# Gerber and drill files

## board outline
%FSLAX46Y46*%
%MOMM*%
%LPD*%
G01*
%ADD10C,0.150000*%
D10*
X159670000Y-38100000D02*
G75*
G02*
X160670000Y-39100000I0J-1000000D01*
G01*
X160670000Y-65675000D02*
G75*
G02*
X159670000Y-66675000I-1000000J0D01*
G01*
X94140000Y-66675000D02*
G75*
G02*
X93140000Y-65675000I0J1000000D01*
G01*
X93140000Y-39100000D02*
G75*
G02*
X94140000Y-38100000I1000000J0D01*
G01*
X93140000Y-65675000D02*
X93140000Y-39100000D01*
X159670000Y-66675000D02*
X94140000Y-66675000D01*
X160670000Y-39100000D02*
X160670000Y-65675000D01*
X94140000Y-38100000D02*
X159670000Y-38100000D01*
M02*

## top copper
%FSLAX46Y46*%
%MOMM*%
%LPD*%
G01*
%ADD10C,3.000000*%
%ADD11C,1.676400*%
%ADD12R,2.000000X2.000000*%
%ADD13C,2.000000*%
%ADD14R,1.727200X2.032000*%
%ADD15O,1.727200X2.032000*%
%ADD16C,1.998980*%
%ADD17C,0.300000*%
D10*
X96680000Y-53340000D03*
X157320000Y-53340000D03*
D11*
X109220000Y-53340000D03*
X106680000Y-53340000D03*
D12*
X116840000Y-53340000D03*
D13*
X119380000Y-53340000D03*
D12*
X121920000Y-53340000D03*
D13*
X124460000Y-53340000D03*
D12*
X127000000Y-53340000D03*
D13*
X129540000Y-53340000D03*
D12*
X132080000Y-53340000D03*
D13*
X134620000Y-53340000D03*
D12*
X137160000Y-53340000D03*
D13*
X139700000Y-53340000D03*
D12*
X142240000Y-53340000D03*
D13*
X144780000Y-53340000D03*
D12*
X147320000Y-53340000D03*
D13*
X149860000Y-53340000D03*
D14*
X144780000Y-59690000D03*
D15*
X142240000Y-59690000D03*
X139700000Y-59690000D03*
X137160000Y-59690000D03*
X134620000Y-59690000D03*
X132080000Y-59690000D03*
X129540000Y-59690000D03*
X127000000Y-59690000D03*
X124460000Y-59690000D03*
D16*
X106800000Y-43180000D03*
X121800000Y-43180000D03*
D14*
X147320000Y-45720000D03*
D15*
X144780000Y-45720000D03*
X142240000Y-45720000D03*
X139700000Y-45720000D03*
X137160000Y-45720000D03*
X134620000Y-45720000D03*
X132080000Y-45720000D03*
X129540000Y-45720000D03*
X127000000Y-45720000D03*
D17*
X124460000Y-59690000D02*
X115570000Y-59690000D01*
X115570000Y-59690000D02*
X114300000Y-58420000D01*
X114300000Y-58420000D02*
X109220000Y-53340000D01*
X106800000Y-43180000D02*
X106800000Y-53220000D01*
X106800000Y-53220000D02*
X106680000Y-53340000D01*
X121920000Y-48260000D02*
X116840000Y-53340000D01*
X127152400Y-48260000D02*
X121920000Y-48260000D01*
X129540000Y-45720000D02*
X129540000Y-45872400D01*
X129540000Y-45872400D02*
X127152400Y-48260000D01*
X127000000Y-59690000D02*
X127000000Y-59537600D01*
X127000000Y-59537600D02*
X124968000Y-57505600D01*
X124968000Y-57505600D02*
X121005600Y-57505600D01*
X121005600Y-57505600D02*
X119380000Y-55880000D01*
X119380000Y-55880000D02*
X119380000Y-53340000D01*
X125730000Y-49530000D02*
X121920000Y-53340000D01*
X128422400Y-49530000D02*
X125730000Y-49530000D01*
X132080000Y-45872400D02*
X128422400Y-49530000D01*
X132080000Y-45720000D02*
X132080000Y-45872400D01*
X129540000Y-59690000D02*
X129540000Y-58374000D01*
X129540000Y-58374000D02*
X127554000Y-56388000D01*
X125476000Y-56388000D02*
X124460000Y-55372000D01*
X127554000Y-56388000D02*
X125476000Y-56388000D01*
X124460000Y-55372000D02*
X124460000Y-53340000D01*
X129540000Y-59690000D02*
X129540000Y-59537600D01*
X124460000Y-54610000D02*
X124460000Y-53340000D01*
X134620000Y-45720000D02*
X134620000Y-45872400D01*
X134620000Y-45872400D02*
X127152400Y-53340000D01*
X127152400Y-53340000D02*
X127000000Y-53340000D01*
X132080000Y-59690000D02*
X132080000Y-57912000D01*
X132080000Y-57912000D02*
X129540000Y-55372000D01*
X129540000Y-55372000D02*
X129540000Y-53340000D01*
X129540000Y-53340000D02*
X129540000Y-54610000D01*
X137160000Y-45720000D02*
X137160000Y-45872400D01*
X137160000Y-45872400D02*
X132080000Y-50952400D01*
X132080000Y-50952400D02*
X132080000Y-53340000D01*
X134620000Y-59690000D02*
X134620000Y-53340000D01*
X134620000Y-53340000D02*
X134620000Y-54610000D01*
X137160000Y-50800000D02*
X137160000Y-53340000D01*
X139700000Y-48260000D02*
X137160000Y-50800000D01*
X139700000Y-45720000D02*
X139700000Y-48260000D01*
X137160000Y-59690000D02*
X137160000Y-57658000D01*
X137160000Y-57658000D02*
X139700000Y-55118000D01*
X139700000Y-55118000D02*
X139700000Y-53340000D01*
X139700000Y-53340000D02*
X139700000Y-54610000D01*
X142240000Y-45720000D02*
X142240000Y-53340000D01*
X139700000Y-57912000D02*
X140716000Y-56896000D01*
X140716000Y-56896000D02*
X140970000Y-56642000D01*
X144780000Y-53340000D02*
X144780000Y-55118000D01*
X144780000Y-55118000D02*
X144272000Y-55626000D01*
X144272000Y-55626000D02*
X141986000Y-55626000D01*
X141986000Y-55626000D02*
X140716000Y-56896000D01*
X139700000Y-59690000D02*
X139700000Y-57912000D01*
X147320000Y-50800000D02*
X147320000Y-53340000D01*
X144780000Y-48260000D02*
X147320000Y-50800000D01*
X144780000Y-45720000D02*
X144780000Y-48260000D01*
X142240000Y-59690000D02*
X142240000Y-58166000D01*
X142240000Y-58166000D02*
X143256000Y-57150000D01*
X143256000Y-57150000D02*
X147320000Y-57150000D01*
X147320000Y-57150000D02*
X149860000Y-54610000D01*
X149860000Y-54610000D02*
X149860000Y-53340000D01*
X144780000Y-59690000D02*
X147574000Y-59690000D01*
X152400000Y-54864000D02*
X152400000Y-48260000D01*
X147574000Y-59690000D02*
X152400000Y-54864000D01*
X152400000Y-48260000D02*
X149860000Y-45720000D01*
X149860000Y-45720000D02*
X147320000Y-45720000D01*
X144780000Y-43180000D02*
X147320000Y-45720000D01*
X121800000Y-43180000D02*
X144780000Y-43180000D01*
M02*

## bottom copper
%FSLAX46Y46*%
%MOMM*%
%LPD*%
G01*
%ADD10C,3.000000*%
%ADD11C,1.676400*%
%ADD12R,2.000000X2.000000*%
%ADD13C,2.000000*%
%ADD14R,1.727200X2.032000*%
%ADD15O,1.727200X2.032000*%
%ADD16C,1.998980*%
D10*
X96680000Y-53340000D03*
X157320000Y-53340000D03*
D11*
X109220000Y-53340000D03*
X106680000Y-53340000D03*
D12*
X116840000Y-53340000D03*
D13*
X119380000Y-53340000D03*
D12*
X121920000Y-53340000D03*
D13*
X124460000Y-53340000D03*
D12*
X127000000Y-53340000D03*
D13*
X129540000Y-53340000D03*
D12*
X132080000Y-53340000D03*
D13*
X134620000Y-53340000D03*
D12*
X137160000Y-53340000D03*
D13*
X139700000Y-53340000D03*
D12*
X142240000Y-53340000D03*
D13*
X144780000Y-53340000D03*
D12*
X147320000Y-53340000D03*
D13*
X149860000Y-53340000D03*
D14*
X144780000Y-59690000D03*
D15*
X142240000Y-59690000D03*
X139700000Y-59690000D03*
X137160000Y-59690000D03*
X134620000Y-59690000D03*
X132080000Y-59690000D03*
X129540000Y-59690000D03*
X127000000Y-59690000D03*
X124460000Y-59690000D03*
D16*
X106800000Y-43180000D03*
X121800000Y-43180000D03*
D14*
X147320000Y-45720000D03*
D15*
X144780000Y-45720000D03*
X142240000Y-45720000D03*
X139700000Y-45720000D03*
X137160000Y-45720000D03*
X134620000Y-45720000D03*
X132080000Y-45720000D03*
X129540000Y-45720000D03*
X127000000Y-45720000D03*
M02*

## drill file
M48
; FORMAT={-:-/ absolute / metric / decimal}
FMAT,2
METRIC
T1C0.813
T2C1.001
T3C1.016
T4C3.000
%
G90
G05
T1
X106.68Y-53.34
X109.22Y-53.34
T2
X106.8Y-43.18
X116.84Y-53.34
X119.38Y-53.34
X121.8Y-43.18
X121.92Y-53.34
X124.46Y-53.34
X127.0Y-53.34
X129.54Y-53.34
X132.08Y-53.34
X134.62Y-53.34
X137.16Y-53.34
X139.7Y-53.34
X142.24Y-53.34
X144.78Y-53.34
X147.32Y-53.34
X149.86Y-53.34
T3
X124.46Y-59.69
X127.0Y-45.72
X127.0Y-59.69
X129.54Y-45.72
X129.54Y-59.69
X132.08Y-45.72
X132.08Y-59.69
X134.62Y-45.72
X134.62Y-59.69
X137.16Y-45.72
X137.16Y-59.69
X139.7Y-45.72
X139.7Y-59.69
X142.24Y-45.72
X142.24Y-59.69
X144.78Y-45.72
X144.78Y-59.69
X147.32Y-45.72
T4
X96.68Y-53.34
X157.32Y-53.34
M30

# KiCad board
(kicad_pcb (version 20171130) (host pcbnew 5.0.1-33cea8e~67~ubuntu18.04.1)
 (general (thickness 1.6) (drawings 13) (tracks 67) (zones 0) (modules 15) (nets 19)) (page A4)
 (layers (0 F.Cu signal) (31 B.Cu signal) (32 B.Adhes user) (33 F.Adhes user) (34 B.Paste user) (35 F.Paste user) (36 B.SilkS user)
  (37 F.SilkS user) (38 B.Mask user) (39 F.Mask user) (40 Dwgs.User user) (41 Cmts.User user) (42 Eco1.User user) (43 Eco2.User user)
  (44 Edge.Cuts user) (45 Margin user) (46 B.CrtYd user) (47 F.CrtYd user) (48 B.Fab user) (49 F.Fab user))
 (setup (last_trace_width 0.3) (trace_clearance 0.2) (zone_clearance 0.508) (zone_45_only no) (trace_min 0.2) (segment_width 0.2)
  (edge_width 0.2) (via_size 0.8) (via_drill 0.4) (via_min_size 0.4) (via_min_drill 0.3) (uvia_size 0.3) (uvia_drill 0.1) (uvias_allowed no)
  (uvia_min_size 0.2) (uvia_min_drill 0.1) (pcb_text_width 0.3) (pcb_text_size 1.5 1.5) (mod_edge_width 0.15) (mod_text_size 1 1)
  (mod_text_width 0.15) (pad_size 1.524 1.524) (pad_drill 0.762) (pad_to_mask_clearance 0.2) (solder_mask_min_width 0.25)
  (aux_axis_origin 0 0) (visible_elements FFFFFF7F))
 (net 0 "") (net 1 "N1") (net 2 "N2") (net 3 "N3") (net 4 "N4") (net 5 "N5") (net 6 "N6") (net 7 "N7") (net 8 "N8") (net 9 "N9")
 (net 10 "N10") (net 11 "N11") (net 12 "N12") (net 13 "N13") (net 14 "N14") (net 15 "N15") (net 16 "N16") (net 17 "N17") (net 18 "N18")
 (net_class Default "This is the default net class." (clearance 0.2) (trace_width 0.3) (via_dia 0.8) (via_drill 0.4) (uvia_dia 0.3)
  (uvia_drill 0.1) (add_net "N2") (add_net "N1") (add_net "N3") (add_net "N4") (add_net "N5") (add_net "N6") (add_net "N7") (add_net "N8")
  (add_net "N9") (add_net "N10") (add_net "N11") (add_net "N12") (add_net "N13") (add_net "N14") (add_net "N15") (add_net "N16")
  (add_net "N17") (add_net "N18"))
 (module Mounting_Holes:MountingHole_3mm (layer F.Cu) (at 96.68 53.34)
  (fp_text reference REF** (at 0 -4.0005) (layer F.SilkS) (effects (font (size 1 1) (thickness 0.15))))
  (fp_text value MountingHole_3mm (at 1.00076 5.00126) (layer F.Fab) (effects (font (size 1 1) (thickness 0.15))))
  (pad 1 thru_hole circle (at 0 0) (size 3 3) (drill 3) (layers)))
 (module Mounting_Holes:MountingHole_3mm (layer F.Cu) (at 157.32 53.34)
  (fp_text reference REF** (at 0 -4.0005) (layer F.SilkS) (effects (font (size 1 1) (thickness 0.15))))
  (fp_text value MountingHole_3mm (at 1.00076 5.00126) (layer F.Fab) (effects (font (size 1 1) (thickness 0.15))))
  (pad 1 thru_hole circle (at 0 0) (size 3 3) (drill 3) (layers)))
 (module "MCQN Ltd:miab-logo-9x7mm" (layer B.Cu) (at 154.432 61.722 180)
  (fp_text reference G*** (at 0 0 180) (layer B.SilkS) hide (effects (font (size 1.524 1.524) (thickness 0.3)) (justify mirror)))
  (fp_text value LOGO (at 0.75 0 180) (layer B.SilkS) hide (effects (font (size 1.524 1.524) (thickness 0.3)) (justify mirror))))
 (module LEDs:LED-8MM (layer B.Cu) (at 106.68 53.34)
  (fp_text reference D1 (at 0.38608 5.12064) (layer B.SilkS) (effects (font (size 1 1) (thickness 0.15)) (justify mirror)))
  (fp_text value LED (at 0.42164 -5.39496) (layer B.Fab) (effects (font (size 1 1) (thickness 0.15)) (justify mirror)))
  (pad 2 thru_hole circle (at 2.54 0 180) (size 1.6764 1.6764) (drill 0.8128) (layers *.Cu *.Mask B.SilkS) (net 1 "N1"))
  (pad 1 thru_hole circle (at 0 0 180) (size 1.6764 1.6764) (drill 0.8128) (layers *.Cu *.Mask B.SilkS) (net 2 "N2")))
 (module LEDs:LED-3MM (layer B.Cu) (at 116.84 53.34)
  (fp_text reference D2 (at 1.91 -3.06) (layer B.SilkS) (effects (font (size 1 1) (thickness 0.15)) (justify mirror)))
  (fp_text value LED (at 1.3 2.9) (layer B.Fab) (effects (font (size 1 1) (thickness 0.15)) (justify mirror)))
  (pad 1 thru_hole rect (at 0 0 270) (size 2 2) (drill 1.00076) (layers *.Cu *.Mask B.SilkS) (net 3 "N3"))
  (pad 2 thru_hole circle (at 2.54 0) (size 2 2) (drill 1.00076) (layers *.Cu *.Mask B.SilkS) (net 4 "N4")))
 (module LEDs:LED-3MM (layer B.Cu) (at 121.92 53.34)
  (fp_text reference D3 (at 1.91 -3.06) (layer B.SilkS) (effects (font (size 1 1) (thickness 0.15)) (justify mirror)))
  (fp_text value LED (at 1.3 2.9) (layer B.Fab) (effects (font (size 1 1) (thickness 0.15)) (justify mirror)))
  (pad 1 thru_hole rect (at 0 0 270) (size 2 2) (drill 1.00076) (layers *.Cu *.Mask B.SilkS) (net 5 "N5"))
  (pad 2 thru_hole circle (at 2.54 0) (size 2 2) (drill 1.00076) (layers *.Cu *.Mask B.SilkS) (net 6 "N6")))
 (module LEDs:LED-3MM (layer B.Cu) (at 127 53.34)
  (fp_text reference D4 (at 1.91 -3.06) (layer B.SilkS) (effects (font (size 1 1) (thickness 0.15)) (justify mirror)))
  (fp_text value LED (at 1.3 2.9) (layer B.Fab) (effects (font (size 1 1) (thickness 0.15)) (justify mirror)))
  (pad 1 thru_hole rect (at 0 0 270) (size 2 2) (drill 1.00076) (layers *.Cu *.Mask B.SilkS) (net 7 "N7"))
  (pad 2 thru_hole circle (at 2.54 0) (size 2 2) (drill 1.00076) (layers *.Cu *.Mask B.SilkS) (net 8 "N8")))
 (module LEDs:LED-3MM (layer B.Cu) (at 132.08 53.34)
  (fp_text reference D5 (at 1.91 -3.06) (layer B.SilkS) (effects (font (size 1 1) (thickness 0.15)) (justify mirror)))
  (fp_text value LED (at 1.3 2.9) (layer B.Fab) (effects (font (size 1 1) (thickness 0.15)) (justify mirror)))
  (pad 1 thru_hole rect (at 0 0 270) (size 2 2) (drill 1.00076) (layers *.Cu *.Mask B.SilkS) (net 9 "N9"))
  (pad 2 thru_hole circle (at 2.54 0) (size 2 2) (drill 1.00076) (layers *.Cu *.Mask B.SilkS) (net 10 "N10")))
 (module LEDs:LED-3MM (layer B.Cu) (at 137.16 53.34)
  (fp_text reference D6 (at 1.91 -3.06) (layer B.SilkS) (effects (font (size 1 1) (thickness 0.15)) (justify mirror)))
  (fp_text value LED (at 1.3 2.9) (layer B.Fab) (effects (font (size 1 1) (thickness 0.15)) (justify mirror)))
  (pad 1 thru_hole rect (at 0 0 270) (size 2 2) (drill 1.00076) (layers *.Cu *.Mask B.SilkS) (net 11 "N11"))
  (pad 2 thru_hole circle (at 2.54 0) (size 2 2) (drill 1.00076) (layers *.Cu *.Mask B.SilkS) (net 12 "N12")))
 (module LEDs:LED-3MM (layer B.Cu) (at 142.24 53.34)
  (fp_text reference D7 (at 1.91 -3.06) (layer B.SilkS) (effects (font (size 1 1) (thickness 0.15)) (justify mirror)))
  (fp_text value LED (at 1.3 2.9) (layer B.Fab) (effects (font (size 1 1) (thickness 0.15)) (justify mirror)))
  (pad 1 thru_hole rect (at 0 0 270) (size 2 2) (drill 1.00076) (layers *.Cu *.Mask B.SilkS) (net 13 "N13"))
  (pad 2 thru_hole circle (at 2.54 0) (size 2 2) (drill 1.00076) (layers *.Cu *.Mask B.SilkS) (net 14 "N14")))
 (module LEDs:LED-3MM (layer B.Cu) (at 147.32 53.34)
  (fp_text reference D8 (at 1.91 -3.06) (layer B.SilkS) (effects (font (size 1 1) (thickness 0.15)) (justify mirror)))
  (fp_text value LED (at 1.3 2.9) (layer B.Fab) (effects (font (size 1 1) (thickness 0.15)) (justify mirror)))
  (pad 1 thru_hole rect (at 0 0 270) (size 2 2) (drill 1.00076) (layers *.Cu *.Mask B.SilkS) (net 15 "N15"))
  (pad 2 thru_hole circle (at 2.54 0) (size 2 2) (drill 1.00076) (layers *.Cu *.Mask B.SilkS) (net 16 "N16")))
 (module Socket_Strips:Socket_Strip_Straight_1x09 (layer F.Cu) (at 144.78 59.69 180)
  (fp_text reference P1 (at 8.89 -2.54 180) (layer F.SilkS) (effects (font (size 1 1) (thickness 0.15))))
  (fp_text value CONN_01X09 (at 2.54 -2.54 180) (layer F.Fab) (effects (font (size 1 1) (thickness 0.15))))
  (pad 1 thru_hole rect (at 0 0 180) (size 1.7272 2.032) (drill 1.016) (layers *.Cu *.Mask F.SilkS) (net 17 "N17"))
  (pad 2 thru_hole oval (at 2.54 0 180) (size 1.7272 2.032) (drill 1.016) (layers *.Cu *.Mask F.SilkS) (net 16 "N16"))
  (pad 3 thru_hole oval (at 5.08 0 180) (size 1.7272 2.032) (drill 1.016) (layers *.Cu *.Mask F.SilkS) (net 14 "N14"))
  (pad 4 thru_hole oval (at 7.62 0 180) (size 1.7272 2.032) (drill 1.016) (layers *.Cu *.Mask F.SilkS) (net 12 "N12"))
  (pad 5 thru_hole oval (at 10.16 0 180) (size 1.7272 2.032) (drill 1.016) (layers *.Cu *.Mask F.SilkS) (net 10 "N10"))
  (pad 6 thru_hole oval (at 12.7 0 180) (size 1.7272 2.032) (drill 1.016) (layers *.Cu *.Mask F.SilkS) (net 8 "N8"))
  (pad 7 thru_hole oval (at 15.24 0 180) (size 1.7272 2.032) (drill 1.016) (layers *.Cu *.Mask F.SilkS) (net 6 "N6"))
  (pad 8 thru_hole oval (at 17.78 0 180) (size 1.7272 2.032) (drill 1.016) (layers *.Cu *.Mask F.SilkS) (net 4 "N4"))
  (pad 9 thru_hole oval (at 20.32 0 180) (size 1.7272 2.032) (drill 1.016) (layers *.Cu *.Mask F.SilkS) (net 1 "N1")))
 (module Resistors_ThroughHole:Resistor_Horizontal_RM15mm (layer F.Cu) (at 114.3 43.18)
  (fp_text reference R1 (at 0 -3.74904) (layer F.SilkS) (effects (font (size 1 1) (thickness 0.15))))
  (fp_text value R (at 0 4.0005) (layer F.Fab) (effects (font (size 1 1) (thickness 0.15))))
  (pad 1 thru_hole circle (at -7.5 0) (size 1.99898 1.99898) (drill 1.00076) (layers *.Cu *.SilkS *.Mask) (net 2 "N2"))
  (pad 2 thru_hole circle (at 7.5 0) (size 1.99898 1.99898) (drill 1.00076) (layers *.Cu *.SilkS *.Mask) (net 17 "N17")))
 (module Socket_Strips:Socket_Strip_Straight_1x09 (layer F.Cu) (at 147.32 45.72 180)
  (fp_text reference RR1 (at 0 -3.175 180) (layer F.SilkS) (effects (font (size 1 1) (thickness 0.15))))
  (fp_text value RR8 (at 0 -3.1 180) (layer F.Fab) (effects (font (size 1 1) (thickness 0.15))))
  (pad 1 thru_hole rect (at 0 0 180) (size 1.7272 2.032) (drill 1.016) (layers *.Cu *.Mask F.SilkS) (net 17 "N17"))
  (pad 2 thru_hole oval (at 2.54 0 180) (size 1.7272 2.032) (drill 1.016) (layers *.Cu *.Mask F.SilkS) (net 15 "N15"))
  (pad 3 thru_hole oval (at 5.08 0 180) (size 1.7272 2.032) (drill 1.016) (layers *.Cu *.Mask F.SilkS) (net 13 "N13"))
  (pad 4 thru_hole oval (at 7.62 0 180) (size 1.7272 2.032) (drill 1.016) (layers *.Cu *.Mask F.SilkS) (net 11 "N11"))
  (pad 5 thru_hole oval (at 10.16 0 180) (size 1.7272 2.032) (drill 1.016) (layers *.Cu *.Mask F.SilkS) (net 9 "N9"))
  (pad 6 thru_hole oval (at 12.7 0 180) (size 1.7272 2.032) (drill 1.016) (layers *.Cu *.Mask F.SilkS) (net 7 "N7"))
  (pad 7 thru_hole oval (at 15.24 0 180) (size 1.7272 2.032) (drill 1.016) (layers *.Cu *.Mask F.SilkS) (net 5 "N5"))
  (pad 8 thru_hole oval (at 17.78 0 180) (size 1.7272 2.032) (drill 1.016) (layers *.Cu *.Mask F.SilkS) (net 3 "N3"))
  (pad 9 thru_hole oval (at 20.32 0 180) (size 1.7272 2.032) (drill 1.016) (layers *.Cu *.Mask F.SilkS) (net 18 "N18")))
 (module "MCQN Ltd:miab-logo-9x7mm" (layer F.Cu) (at 99.314 61.722)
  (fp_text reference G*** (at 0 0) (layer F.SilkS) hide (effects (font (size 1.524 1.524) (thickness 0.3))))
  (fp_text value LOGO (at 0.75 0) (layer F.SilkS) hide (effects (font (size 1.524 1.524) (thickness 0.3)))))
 (gr_arc (start 159.67 39.1) (end 159.67 38.1) (angle 90) (layer Edge.Cuts) (width 0.15))
 (gr_arc (start 159.67 65.675) (end 159.67 66.675) (angle -90) (layer Edge.Cuts) (width 0.15))
 (gr_arc (start 94.14 65.675) (end 93.14 65.675) (angle -90) (layer Edge.Cuts) (width 0.15))
 (gr_arc (start 94.14 39.1) (end 93.14 39.1) (angle 90) (layer Edge.Cuts) (width 0.15))
 (gr_line (start 93.14 65.675) (end 93.14 39.1) (layer Edge.Cuts) (width 0.15))
 (gr_line (start 159.67 66.675) (end 94.14 66.675) (layer Edge.Cuts) (width 0.15))
 (gr_line (start 160.67 39.1) (end 160.67 65.675) (layer Edge.Cuts) (width 0.15))
 (gr_line (start 94.14 38.1) (end 159.67 38.1) (layer Edge.Cuts) (width 0.15))
 (segment (start 124.46 59.69) (end 115.57 59.69) (width 0.3) (layer F.Cu) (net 1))
 (segment (start 115.57 59.69) (end 114.3 58.42) (width 0.3) (layer F.Cu) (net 1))
 (segment (start 114.3 58.42) (end 109.22 53.34) (width 0.3) (layer F.Cu) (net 1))
 (segment (start 106.8 43.18) (end 106.8 53.22) (width 0.3) (layer F.Cu) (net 2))
 (segment (start 106.8 53.22) (end 106.68 53.34) (width 0.3) (layer F.Cu) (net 2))
 (segment (start 121.92 48.26) (end 116.84 53.34) (width 0.3) (layer F.Cu) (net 3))
 (segment (start 127.1524 48.26) (end 121.92 48.26) (width 0.3) (layer F.Cu) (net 3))
 (segment (start 129.54 45.72) (end 129.54 45.8724) (width 0.3) (layer F.Cu) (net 3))
 (segment (start 129.54 45.8724) (end 127.1524 48.26) (width 0.3) (layer F.Cu) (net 3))
 (segment (start 127 59.69) (end 127 59.5376) (width 0.3) (layer F.Cu) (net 4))
 (segment (start 127 59.5376) (end 124.968 57.5056) (width 0.3) (layer F.Cu) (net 4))
 (segment (start 124.968 57.5056) (end 121.0056 57.5056) (width 0.3) (layer F.Cu) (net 4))
 (segment (start 121.0056 57.5056) (end 119.38 55.88) (width 0.3) (layer F.Cu) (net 4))
 (segment (start 119.38 55.88) (end 119.38 53.34) (width 0.3) (layer F.Cu) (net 4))
 (segment (start 125.73 49.53) (end 121.92 53.34) (width 0.3) (layer F.Cu) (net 5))
 (segment (start 128.4224 49.53) (end 125.73 49.53) (width 0.3) (layer F.Cu) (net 5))
 (segment (start 132.08 45.8724) (end 128.4224 49.53) (width 0.3) (layer F.Cu) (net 5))
 (segment (start 132.08 45.72) (end 132.08 45.8724) (width 0.3) (layer F.Cu) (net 5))
 (segment (start 129.54 59.69) (end 129.54 58.374) (width 0.3) (layer F.Cu) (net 6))
 (segment (start 129.54 58.374) (end 127.554 56.388) (width 0.3) (layer F.Cu) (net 6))
 (segment (start 125.476 56.388) (end 124.46 55.372) (width 0.3) (layer F.Cu) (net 6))
 (segment (start 127.554 56.388) (end 125.476 56.388) (width 0.3) (layer F.Cu) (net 6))
 (segment (start 124.46 55.372) (end 124.46 53.34) (width 0.3) (layer F.Cu) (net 6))
 (segment (start 129.54 59.69) (end 129.54 59.5376) (width 0.3) (layer F.Cu) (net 6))
 (segment (start 124.46 54.61) (end 124.46 53.34) (width 0.3) (layer F.Cu) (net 6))
 (segment (start 134.62 45.72) (end 134.62 45.8724) (width 0.3) (layer F.Cu) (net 7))
 (segment (start 134.62 45.8724) (end 127.1524 53.34) (width 0.3) (layer F.Cu) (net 7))
 (segment (start 127.1524 53.34) (end 127 53.34) (width 0.3) (layer F.Cu) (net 7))
 (segment (start 132.08 59.69) (end 132.08 57.912) (width 0.3) (layer F.Cu) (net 8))
 (segment (start 132.08 57.912) (end 129.54 55.372) (width 0.3) (layer F.Cu) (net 8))
 (segment (start 129.54 55.372) (end 129.54 53.34) (width 0.3) (layer F.Cu) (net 8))
 (segment (start 129.54 53.34) (end 129.54 54.61) (width 0.3) (layer F.Cu) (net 8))
 (segment (start 137.16 45.72) (end 137.16 45.8724) (width 0.3) (layer F.Cu) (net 9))
 (segment (start 137.16 45.8724) (end 132.08 50.9524) (width 0.3) (layer F.Cu) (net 9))
 (segment (start 132.08 50.9524) (end 132.08 53.34) (width 0.3) (layer F.Cu) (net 9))
 (segment (start 134.62 59.69) (end 134.62 53.34) (width 0.3) (layer F.Cu) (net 10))
 (segment (start 134.62 53.34) (end 134.62 54.61) (width 0.3) (layer F.Cu) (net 10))
 (segment (start 137.16 50.8) (end 137.16 53.34) (width 0.3) (layer F.Cu) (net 11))
 (segment (start 139.7 48.26) (end 137.16 50.8) (width 0.3) (layer F.Cu) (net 11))
 (segment (start 139.7 45.72) (end 139.7 48.26) (width 0.3) (layer F.Cu) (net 11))
 (segment (start 137.16 59.69) (end 137.16 57.658) (width 0.3) (layer F.Cu) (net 12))
 (segment (start 137.16 57.658) (end 139.7 55.118) (width 0.3) (layer F.Cu) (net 12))
 (segment (start 139.7 55.118) (end 139.7 53.34) (width 0.3) (layer F.Cu) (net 12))
 (segment (start 139.7 53.34) (end 139.7 54.61) (width 0.3) (layer F.Cu) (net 12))
 (segment (start 142.24 45.72) (end 142.24 53.34) (width 0.3) (layer F.Cu) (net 13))
 (segment (start 139.7 57.912) (end 140.716 56.896) (width 0.3) (layer F.Cu) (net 14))
 (segment (start 140.716 56.896) (end 140.97 56.642) (width 0.3) (layer F.Cu) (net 14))
 (segment (start 144.78 53.34) (end 144.78 55.118) (width 0.3) (layer F.Cu) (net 14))
 (segment (start 144.78 55.118) (end 144.272 55.626) (width 0.3) (layer F.Cu) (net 14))
 (segment (start 144.272 55.626) (end 141.986 55.626) (width 0.3) (layer F.Cu) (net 14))
 (segment (start 141.986 55.626) (end 140.716 56.896) (width 0.3) (layer F.Cu) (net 14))
 (segment (start 139.7 59.69) (end 139.7 57.912) (width 0.3) (layer F.Cu) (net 14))
 (segment (start 147.32 50.8) (end 147.32 53.34) (width 0.3) (layer F.Cu) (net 15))
 (segment (start 144.78 48.26) (end 147.32 50.8) (width 0.3) (layer F.Cu) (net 15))
 (segment (start 144.78 45.72) (end 144.78 48.26) (width 0.3) (layer F.Cu) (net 15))
 (segment (start 142.24 59.69) (end 142.24 58.166) (width 0.3) (layer F.Cu) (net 16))
 (segment (start 142.24 58.166) (end 143.256 57.15) (width 0.3) (layer F.Cu) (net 16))
 (segment (start 143.256 57.15) (end 147.32 57.15) (width 0.3) (layer F.Cu) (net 16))
 (segment (start 147.32 57.15) (end 149.86 54.61) (width 0.3) (layer F.Cu) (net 16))
 (segment (start 149.86 54.61) (end 149.86 53.34) (width 0.3) (layer F.Cu) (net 16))
 (segment (start 144.78 59.69) (end 147.574 59.69) (width 0.3) (layer F.Cu) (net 17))
 (segment (start 152.4 54.864) (end 152.4 48.26) (width 0.3) (layer F.Cu) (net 17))
 (segment (start 147.574 59.69) (end 152.4 54.864) (width 0.3) (layer F.Cu) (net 17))
 (segment (start 152.4 48.26) (end 149.86 45.72) (width 0.3) (layer F.Cu) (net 17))
 (segment (start 149.86 45.72) (end 147.32 45.72) (width 0.3) (layer F.Cu) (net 17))
 (segment (start 144.78 43.18) (end 147.32 45.72) (width 0.3) (layer F.Cu) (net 17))
 (segment (start 121.8 43.18) (end 144.78 43.18) (width 0.3) (layer F.Cu) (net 17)))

